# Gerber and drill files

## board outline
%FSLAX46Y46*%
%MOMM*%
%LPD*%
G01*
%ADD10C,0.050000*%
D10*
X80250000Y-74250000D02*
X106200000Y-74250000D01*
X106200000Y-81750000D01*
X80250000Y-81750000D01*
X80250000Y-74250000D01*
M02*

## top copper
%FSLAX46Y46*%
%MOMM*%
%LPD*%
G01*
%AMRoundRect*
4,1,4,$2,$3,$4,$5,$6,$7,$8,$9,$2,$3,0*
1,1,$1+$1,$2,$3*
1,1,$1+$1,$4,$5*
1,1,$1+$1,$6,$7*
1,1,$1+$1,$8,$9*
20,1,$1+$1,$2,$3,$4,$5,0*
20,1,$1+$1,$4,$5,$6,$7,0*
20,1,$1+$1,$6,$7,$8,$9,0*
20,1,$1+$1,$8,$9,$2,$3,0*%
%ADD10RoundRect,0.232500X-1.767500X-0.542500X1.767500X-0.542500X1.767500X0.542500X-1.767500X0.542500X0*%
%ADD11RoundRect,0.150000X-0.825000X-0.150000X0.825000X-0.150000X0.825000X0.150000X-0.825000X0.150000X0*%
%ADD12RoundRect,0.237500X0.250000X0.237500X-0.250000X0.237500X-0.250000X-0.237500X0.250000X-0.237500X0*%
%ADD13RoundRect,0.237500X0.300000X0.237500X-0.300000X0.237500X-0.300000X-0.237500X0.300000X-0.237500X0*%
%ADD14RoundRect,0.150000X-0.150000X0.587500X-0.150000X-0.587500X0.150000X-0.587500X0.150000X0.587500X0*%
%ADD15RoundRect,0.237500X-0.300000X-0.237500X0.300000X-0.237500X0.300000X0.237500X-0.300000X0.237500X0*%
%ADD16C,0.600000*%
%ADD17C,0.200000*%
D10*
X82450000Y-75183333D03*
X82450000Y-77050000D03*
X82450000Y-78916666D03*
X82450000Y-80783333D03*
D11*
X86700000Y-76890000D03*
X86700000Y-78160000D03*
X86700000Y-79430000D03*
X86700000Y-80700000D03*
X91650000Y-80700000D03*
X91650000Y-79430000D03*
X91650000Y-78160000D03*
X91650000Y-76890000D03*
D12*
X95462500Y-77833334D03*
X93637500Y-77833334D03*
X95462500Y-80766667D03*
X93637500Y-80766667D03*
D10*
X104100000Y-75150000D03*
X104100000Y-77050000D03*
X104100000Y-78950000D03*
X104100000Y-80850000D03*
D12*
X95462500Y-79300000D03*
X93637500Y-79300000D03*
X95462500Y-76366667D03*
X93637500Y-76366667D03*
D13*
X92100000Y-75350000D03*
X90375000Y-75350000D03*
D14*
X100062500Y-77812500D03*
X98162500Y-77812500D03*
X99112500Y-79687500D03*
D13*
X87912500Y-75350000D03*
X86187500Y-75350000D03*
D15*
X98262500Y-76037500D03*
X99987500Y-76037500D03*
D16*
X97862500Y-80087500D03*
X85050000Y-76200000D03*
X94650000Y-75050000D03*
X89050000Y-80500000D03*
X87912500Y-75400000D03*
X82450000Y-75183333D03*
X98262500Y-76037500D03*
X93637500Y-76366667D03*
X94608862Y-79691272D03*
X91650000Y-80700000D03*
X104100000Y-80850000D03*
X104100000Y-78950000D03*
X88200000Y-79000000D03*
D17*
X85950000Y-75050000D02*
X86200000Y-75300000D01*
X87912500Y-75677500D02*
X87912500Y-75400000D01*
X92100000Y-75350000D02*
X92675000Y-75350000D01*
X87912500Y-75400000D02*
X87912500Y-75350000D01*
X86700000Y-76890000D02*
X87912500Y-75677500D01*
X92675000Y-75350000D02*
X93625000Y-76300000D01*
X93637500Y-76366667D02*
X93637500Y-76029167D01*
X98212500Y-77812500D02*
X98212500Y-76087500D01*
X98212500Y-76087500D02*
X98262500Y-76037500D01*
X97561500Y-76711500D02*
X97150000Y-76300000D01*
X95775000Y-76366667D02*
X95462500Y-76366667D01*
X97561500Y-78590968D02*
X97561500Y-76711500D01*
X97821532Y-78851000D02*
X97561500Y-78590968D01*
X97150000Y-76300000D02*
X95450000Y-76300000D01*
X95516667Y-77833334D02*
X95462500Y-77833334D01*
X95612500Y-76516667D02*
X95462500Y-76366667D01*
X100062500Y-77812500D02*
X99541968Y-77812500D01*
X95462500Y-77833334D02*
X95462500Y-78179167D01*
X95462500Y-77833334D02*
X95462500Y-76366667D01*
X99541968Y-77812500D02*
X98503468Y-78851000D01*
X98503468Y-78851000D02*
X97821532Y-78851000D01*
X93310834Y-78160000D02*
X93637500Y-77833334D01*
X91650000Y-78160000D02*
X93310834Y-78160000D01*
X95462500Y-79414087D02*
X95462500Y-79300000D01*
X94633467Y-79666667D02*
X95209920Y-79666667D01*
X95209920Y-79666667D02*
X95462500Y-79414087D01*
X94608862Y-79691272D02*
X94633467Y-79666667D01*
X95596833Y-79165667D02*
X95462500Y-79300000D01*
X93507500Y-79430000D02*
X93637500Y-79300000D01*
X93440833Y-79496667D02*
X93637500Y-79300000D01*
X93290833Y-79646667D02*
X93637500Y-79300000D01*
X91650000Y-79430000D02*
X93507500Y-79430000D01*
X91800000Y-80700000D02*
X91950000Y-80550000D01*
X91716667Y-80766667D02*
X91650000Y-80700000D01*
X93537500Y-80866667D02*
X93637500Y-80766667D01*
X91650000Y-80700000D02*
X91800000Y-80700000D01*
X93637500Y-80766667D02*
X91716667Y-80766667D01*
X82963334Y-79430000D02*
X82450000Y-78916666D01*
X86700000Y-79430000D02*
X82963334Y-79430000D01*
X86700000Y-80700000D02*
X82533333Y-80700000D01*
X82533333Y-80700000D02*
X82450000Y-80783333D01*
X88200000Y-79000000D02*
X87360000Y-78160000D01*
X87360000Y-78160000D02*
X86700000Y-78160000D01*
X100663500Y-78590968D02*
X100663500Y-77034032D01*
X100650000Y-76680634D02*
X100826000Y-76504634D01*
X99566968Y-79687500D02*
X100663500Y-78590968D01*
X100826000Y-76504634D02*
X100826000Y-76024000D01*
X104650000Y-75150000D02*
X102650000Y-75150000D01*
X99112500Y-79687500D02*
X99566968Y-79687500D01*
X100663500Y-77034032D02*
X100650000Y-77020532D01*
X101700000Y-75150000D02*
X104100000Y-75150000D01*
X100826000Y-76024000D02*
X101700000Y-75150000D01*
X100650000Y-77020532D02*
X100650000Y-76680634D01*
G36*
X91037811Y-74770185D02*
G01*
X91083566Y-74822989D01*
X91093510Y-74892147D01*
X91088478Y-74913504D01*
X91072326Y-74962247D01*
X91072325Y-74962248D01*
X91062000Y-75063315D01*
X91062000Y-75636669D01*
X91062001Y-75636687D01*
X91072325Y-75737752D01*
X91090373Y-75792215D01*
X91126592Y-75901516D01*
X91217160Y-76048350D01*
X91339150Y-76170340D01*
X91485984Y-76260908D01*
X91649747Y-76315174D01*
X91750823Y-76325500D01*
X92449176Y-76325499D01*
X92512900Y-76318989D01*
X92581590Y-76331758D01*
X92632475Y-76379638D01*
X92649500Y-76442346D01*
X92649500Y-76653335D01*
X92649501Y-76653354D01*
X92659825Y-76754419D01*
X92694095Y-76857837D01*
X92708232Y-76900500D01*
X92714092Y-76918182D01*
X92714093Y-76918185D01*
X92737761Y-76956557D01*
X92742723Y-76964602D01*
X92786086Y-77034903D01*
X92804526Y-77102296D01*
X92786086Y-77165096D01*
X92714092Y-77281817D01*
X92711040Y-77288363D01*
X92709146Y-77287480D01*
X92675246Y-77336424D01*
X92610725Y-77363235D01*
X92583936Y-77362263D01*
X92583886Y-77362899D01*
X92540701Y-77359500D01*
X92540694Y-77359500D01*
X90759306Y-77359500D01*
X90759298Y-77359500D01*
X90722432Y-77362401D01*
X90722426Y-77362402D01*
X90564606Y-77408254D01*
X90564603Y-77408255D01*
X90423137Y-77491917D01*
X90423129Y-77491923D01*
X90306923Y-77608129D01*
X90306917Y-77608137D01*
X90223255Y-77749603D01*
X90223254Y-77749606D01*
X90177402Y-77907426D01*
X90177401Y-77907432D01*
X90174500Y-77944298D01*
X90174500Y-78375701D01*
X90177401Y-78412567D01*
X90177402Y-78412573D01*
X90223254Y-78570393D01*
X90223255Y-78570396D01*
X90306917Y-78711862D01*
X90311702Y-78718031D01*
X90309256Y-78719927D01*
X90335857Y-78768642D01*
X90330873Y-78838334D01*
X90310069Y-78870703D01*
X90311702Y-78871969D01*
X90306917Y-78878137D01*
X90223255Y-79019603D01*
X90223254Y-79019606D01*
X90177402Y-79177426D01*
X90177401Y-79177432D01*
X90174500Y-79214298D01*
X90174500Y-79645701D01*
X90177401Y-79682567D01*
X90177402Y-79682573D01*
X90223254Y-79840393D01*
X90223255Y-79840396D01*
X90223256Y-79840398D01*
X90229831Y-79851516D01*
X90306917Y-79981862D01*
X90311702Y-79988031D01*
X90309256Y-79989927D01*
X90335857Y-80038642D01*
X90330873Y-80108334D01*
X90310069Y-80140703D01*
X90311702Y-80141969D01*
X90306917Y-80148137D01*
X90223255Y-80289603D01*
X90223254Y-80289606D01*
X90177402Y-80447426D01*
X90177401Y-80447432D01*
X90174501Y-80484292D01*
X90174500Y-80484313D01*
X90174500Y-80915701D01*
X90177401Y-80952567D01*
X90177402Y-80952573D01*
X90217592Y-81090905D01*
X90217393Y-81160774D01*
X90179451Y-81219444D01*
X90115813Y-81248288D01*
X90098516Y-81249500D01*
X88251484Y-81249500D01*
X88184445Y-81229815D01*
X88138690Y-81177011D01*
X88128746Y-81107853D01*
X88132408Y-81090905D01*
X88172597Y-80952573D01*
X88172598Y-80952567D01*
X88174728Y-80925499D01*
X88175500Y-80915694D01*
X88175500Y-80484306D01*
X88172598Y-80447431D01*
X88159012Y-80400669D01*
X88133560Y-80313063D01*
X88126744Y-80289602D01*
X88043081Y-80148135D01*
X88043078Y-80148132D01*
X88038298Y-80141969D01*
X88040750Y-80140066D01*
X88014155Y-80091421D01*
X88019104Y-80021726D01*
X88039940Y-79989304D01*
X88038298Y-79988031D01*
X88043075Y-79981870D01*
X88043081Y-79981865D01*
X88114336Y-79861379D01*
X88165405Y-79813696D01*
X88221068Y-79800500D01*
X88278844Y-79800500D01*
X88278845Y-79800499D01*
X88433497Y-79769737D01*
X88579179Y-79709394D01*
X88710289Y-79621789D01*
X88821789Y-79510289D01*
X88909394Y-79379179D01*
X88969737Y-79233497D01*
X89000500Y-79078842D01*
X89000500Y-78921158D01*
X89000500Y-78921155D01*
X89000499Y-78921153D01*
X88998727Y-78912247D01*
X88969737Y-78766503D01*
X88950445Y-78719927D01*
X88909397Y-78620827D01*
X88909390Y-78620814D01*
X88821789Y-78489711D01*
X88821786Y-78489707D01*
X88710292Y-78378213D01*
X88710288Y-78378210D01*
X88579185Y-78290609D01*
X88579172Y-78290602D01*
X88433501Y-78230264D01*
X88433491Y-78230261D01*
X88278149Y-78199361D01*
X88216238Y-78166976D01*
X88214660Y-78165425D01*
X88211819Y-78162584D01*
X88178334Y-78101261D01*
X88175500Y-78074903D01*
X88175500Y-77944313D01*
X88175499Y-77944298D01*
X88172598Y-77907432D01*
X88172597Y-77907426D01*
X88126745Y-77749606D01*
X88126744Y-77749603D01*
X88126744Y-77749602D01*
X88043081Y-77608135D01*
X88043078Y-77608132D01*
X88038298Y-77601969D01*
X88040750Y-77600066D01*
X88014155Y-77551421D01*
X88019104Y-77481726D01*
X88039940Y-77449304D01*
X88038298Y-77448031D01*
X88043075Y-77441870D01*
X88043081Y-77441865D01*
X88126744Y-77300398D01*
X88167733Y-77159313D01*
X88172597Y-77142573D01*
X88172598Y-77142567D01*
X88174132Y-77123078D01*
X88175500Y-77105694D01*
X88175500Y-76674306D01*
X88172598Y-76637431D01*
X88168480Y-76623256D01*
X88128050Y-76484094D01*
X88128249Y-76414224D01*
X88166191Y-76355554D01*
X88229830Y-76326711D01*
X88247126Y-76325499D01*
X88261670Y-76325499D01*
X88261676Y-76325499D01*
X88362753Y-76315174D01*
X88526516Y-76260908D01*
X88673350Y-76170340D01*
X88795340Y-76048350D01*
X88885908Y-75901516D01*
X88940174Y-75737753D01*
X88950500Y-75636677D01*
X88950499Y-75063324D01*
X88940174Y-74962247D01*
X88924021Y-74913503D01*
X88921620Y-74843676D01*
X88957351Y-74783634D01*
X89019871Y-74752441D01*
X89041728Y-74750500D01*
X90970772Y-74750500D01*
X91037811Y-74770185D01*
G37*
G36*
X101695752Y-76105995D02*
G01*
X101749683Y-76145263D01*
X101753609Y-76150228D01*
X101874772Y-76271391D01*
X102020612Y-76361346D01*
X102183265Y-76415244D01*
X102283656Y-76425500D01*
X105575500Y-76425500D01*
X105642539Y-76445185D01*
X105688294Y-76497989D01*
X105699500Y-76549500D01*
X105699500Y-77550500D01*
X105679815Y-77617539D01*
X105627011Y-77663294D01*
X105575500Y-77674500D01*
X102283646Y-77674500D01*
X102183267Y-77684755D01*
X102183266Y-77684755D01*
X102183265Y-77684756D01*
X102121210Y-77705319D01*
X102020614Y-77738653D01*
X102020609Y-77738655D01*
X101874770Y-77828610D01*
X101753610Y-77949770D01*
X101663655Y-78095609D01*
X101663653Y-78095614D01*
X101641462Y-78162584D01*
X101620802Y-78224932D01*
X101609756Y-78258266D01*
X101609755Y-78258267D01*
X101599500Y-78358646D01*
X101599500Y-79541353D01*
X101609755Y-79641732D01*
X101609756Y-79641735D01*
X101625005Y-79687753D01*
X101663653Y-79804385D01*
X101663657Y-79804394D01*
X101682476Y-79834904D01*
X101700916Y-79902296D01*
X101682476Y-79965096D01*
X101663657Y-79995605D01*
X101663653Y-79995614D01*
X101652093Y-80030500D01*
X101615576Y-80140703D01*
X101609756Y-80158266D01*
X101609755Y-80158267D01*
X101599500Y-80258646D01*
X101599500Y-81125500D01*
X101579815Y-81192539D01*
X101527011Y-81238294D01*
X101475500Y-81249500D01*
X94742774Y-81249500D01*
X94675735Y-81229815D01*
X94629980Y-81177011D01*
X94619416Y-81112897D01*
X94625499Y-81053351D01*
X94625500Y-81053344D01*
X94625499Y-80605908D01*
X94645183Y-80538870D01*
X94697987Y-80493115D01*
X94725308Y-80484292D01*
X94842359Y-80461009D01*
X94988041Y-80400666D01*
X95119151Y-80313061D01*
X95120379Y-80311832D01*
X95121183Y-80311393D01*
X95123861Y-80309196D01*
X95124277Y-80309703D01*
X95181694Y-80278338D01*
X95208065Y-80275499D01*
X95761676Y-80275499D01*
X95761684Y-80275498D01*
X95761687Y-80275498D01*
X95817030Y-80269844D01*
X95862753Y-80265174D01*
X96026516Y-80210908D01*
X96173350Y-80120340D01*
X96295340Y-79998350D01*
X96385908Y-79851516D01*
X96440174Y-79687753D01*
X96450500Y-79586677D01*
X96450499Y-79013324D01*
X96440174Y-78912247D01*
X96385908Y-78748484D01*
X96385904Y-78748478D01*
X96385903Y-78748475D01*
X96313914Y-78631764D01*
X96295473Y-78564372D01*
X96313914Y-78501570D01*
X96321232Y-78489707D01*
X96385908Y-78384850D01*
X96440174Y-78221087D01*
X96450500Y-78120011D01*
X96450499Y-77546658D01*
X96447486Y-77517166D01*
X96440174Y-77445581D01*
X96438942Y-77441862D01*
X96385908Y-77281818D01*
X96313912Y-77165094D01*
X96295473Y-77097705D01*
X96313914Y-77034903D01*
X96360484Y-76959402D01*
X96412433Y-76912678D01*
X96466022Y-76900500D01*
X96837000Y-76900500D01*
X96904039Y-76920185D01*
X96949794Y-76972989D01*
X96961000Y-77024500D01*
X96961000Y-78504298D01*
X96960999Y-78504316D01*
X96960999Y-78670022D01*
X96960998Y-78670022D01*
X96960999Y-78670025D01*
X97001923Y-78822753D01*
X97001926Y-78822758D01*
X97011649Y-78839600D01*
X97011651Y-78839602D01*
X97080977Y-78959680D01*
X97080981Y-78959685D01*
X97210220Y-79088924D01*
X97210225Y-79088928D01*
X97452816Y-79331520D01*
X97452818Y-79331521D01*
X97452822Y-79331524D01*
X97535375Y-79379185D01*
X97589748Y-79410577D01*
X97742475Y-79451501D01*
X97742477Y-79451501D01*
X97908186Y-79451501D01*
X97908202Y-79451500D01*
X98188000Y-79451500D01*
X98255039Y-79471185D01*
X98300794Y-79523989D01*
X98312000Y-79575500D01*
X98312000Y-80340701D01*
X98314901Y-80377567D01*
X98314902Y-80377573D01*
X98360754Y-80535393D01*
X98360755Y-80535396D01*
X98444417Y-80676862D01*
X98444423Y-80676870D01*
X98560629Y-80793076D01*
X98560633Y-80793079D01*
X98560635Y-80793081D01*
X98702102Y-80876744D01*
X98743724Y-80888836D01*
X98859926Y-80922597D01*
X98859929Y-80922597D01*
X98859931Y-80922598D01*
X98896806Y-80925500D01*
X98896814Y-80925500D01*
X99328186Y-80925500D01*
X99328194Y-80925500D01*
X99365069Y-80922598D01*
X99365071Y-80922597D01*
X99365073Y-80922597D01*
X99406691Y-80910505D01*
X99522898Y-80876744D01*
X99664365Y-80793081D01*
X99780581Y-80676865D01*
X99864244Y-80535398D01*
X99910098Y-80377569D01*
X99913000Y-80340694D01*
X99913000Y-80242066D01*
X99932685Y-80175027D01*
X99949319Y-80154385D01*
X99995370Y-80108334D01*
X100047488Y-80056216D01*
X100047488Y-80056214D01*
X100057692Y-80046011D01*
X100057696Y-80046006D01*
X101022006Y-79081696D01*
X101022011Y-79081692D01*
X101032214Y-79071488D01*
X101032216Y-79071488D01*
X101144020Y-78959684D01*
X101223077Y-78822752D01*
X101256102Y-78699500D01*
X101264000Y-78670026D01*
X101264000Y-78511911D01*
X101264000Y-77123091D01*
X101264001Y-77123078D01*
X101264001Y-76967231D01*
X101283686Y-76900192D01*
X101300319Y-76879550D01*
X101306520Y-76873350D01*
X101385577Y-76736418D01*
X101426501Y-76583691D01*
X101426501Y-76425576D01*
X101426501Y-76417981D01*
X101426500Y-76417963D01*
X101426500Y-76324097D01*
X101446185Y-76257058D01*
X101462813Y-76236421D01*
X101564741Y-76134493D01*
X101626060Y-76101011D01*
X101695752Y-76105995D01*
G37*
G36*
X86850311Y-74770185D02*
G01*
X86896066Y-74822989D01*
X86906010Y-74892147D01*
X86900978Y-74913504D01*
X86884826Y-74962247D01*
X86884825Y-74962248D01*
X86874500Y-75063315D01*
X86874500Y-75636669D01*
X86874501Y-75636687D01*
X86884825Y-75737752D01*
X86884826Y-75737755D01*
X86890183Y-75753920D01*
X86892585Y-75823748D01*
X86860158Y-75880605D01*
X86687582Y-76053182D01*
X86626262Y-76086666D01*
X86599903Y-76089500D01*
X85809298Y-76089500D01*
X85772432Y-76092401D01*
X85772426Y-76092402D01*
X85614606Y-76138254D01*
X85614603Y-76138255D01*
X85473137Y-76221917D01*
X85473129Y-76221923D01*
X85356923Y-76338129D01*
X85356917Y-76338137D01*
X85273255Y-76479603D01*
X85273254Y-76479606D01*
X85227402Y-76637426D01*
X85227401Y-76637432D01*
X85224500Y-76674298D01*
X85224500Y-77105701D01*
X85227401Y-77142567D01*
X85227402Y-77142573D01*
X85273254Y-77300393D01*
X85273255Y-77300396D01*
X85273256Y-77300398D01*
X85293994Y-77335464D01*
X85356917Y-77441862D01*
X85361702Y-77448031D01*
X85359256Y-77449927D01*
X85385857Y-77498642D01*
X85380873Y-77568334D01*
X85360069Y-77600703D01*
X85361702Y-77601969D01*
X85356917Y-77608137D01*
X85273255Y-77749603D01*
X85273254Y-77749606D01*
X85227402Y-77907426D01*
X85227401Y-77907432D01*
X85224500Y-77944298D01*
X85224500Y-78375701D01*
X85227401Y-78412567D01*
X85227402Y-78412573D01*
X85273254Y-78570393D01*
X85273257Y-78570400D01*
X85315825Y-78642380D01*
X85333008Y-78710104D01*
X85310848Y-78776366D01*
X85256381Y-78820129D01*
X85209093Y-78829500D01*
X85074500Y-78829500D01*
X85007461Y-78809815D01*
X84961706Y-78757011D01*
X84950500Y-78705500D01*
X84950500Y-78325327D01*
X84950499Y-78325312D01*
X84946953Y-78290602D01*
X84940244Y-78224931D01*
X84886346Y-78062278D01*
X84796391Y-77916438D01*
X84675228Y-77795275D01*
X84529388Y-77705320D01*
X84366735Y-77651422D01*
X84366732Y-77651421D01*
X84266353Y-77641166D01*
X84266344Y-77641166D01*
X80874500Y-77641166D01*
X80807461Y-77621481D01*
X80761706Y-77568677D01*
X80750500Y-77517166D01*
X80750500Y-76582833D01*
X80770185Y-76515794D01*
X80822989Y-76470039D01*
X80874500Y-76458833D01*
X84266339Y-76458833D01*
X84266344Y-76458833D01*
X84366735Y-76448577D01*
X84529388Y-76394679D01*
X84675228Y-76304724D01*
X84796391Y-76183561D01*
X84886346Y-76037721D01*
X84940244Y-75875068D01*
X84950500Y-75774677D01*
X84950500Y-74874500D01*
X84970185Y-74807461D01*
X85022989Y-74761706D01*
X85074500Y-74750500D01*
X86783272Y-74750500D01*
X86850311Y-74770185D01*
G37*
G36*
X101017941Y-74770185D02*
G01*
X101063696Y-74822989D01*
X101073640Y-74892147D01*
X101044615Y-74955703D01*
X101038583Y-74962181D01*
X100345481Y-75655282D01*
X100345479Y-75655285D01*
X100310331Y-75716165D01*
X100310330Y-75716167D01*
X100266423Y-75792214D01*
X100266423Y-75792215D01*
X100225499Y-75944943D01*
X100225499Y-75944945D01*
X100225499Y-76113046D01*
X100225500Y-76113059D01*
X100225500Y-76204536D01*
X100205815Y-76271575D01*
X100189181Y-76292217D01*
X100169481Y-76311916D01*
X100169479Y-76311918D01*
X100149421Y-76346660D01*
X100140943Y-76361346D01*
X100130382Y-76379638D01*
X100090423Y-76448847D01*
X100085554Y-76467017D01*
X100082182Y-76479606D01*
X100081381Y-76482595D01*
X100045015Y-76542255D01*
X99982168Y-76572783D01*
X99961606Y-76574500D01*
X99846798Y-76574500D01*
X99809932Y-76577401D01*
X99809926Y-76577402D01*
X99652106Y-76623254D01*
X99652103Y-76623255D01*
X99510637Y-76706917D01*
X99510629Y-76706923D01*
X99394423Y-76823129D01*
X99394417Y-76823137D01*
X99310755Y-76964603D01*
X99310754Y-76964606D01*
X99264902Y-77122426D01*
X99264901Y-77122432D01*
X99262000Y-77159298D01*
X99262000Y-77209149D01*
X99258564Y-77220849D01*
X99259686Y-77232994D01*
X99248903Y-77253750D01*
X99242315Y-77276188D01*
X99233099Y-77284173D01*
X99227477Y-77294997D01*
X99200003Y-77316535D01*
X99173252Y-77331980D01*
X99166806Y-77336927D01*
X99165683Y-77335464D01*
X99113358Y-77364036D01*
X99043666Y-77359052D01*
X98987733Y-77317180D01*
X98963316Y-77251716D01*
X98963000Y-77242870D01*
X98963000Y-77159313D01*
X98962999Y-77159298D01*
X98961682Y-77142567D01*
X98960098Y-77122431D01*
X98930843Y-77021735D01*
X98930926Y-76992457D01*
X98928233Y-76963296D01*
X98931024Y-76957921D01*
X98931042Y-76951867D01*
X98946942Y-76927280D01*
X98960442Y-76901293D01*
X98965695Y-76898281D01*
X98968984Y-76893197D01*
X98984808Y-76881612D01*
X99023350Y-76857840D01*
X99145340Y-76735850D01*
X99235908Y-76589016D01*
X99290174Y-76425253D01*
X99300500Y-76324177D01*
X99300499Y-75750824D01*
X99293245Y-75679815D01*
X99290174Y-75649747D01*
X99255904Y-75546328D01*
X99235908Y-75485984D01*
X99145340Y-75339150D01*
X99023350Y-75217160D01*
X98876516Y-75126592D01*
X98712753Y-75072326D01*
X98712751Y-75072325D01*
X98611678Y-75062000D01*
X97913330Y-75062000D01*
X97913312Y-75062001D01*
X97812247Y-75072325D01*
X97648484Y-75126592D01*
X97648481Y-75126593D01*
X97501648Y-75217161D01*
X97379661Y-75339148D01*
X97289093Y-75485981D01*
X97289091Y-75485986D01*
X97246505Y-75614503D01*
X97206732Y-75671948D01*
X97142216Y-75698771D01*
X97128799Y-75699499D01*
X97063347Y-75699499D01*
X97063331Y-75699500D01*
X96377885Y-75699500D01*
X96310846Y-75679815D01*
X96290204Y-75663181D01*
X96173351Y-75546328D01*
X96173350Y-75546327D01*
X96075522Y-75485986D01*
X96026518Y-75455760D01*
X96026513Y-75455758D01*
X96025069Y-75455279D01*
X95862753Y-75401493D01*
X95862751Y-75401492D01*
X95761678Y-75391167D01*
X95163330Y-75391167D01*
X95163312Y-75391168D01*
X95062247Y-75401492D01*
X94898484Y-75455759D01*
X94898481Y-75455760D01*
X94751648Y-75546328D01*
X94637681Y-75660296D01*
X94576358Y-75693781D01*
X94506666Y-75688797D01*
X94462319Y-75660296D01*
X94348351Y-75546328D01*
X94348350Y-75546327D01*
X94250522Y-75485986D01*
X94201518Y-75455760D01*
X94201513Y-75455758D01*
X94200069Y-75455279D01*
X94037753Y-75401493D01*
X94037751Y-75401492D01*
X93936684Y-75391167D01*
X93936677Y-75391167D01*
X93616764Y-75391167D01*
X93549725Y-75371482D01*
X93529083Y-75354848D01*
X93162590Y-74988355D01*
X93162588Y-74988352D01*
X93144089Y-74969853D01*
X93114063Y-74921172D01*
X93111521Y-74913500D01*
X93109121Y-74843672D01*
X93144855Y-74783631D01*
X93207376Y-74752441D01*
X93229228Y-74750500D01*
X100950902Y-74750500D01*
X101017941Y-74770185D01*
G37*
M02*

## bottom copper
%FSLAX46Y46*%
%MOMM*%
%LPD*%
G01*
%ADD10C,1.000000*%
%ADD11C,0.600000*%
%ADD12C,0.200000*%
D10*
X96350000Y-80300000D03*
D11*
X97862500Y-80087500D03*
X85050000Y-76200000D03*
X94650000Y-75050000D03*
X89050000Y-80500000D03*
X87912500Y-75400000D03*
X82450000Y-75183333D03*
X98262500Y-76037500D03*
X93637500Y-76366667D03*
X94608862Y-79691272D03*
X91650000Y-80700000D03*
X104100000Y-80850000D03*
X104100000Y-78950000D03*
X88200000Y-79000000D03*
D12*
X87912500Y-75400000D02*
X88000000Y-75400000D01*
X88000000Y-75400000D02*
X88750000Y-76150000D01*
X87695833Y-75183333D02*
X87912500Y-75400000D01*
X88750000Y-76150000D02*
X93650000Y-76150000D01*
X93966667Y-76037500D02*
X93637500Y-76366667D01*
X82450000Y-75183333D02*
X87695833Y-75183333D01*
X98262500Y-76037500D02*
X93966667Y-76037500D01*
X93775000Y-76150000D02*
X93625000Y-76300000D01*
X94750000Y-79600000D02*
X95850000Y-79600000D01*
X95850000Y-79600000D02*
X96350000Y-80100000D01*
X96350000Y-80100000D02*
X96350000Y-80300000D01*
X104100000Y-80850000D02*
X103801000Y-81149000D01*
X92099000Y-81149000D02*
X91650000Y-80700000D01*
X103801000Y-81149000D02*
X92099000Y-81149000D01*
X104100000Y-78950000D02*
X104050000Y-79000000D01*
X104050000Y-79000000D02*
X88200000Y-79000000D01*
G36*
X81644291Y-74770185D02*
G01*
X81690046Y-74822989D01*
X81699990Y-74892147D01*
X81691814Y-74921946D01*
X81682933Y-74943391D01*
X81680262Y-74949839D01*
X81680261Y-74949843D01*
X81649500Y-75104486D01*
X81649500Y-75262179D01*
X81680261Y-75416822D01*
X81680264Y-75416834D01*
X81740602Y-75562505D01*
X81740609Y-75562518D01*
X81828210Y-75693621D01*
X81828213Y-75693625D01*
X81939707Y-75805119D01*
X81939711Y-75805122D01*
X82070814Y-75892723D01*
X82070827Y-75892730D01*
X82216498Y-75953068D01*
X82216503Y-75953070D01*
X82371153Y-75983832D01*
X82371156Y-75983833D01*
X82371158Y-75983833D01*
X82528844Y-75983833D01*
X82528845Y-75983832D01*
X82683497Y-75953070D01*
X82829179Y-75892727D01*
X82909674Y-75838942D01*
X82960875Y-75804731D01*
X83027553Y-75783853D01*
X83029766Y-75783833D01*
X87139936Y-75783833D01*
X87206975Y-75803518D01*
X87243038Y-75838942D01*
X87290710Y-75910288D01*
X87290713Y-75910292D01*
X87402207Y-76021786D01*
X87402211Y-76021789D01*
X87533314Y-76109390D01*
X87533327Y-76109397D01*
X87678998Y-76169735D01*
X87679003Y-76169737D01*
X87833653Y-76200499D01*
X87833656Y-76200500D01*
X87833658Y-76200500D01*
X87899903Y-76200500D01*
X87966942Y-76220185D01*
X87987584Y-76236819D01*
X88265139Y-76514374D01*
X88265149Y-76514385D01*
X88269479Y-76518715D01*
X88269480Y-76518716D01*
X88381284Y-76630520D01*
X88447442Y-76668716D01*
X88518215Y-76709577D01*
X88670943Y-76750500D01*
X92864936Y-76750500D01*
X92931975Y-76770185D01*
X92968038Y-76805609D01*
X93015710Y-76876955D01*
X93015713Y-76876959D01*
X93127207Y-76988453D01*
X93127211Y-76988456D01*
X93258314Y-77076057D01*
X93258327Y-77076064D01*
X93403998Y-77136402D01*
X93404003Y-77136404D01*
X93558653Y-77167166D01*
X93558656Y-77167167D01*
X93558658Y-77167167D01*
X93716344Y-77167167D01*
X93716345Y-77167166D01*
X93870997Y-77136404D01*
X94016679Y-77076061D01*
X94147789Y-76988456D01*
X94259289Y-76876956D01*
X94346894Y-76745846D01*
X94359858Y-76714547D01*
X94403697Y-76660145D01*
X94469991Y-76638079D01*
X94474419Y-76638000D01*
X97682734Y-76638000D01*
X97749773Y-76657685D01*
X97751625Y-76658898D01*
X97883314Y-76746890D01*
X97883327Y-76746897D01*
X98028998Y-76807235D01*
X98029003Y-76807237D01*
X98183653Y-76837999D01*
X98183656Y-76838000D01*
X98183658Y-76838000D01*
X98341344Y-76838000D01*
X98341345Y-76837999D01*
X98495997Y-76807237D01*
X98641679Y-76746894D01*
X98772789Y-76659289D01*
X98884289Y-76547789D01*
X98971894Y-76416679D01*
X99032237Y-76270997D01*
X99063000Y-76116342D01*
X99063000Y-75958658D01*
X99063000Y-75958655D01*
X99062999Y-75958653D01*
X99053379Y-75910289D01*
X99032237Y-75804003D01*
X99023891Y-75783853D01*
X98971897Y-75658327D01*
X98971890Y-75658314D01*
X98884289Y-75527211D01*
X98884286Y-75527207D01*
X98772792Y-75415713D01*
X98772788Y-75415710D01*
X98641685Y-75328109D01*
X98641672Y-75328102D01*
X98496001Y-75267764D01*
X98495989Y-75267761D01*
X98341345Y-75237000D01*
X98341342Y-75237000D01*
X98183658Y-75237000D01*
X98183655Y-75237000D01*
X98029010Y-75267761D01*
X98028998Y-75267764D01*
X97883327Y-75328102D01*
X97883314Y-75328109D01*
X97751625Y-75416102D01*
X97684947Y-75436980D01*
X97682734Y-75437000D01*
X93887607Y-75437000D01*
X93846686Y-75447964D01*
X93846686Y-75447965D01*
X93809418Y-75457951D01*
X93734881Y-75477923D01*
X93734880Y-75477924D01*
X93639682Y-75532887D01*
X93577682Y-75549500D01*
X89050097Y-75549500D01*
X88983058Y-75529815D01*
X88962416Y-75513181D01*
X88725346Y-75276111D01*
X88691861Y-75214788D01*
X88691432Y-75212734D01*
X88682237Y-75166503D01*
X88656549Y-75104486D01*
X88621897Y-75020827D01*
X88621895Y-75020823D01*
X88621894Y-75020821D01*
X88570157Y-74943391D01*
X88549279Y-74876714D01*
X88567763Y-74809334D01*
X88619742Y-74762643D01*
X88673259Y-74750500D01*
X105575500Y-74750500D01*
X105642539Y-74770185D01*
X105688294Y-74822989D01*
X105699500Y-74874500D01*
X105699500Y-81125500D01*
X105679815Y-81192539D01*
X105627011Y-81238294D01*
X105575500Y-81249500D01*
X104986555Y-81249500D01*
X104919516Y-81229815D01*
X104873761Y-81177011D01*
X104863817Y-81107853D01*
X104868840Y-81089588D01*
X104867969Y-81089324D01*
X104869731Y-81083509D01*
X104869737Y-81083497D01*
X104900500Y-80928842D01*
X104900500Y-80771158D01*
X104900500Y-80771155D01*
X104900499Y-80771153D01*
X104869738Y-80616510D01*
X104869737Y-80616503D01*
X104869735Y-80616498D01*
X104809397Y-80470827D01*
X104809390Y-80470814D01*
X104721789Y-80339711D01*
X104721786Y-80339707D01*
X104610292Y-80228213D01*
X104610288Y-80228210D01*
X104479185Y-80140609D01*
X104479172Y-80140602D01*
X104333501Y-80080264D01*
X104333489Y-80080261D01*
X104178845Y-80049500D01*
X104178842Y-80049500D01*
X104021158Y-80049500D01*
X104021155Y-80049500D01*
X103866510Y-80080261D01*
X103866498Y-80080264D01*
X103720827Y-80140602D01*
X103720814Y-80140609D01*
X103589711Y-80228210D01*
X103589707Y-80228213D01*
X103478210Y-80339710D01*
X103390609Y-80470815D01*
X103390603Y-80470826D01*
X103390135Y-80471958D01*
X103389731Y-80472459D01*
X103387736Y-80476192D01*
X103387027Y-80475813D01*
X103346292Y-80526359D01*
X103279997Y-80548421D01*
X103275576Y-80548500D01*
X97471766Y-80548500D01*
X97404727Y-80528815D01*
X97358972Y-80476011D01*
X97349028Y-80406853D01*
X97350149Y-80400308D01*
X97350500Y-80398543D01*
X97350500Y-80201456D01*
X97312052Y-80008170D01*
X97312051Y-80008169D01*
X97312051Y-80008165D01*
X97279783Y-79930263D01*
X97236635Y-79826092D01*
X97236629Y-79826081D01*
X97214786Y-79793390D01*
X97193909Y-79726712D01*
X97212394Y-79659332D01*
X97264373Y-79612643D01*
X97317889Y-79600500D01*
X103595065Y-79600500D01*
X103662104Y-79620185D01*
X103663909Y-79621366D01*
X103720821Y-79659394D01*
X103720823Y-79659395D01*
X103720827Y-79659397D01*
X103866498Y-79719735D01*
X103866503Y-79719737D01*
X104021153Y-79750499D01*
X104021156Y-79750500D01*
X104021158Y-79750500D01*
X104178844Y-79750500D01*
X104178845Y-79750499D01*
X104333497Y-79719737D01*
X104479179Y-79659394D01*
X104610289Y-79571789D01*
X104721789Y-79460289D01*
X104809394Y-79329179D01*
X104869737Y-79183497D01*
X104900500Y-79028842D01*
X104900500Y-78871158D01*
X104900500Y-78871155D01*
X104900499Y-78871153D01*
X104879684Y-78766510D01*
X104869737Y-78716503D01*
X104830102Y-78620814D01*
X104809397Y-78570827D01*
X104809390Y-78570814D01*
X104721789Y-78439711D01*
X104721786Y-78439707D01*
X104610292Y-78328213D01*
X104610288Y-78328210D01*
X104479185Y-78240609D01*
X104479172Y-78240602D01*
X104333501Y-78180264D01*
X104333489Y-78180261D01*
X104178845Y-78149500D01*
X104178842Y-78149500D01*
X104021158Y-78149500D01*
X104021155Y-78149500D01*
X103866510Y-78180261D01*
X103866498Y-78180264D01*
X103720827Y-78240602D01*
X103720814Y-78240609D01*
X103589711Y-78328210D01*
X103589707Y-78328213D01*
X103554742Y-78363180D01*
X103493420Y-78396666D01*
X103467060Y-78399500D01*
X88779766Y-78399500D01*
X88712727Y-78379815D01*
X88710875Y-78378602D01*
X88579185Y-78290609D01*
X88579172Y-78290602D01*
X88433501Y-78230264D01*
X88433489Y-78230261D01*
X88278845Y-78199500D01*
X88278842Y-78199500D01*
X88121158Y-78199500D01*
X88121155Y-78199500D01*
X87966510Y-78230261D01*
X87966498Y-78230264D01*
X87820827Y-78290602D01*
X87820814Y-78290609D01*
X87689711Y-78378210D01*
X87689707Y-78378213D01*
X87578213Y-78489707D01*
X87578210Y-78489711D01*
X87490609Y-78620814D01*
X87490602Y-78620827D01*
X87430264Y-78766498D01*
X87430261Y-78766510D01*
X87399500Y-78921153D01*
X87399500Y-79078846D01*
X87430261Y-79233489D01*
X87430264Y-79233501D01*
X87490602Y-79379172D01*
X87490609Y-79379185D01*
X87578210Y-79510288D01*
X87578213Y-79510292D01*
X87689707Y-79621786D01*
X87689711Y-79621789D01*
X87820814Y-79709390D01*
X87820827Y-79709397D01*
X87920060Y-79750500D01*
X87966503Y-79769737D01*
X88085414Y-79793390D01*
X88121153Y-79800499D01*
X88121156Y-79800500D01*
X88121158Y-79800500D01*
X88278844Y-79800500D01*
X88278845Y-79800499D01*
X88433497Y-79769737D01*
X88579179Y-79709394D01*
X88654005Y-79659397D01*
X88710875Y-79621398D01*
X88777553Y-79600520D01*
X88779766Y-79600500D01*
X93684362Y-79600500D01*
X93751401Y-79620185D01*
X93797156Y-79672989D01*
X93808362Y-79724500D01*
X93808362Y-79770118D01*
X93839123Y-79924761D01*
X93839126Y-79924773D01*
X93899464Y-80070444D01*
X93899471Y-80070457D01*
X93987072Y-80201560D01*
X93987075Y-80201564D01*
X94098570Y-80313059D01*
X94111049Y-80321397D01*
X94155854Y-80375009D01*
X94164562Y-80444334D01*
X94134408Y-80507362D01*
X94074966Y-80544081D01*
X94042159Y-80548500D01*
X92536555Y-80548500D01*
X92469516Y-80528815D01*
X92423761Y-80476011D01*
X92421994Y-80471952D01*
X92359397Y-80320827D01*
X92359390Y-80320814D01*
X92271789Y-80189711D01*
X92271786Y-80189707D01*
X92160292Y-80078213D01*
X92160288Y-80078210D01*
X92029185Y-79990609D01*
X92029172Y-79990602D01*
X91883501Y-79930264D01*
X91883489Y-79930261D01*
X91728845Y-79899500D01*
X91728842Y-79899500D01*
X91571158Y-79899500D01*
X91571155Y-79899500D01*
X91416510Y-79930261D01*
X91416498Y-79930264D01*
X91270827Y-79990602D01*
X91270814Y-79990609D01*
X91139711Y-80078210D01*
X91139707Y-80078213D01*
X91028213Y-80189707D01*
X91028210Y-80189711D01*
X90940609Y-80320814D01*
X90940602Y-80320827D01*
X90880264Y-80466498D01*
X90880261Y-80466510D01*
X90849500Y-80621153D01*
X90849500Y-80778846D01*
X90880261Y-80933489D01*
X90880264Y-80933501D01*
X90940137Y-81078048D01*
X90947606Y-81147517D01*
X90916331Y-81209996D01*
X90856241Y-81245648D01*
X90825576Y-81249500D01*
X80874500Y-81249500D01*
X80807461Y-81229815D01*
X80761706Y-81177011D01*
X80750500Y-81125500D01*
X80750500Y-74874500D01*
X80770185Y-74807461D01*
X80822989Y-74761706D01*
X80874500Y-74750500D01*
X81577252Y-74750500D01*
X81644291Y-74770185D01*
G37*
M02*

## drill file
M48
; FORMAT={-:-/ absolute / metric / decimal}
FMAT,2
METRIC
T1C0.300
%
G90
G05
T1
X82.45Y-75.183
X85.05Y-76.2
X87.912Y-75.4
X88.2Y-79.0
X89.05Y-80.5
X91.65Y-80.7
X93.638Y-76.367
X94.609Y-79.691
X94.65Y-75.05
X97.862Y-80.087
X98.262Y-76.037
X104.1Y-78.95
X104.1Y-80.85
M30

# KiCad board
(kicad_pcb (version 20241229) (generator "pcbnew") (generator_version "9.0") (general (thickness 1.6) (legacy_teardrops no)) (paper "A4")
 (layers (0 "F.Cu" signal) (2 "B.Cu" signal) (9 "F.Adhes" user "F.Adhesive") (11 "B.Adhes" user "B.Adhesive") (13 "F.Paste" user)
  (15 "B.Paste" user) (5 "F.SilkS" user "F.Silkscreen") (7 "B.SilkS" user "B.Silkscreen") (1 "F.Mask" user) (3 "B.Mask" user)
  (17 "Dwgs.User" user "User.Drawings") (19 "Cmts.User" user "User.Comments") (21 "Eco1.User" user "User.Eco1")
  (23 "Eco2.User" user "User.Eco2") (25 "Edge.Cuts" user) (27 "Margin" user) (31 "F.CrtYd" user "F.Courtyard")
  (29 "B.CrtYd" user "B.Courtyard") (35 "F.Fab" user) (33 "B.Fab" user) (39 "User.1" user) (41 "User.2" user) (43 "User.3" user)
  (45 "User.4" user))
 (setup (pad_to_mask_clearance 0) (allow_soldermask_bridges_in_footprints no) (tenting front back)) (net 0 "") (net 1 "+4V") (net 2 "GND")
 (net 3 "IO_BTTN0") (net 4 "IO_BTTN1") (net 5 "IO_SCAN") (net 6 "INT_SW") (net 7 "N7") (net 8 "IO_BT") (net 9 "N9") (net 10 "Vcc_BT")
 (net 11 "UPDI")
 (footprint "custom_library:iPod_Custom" (layer "F.Cu") (at 83 82.433333)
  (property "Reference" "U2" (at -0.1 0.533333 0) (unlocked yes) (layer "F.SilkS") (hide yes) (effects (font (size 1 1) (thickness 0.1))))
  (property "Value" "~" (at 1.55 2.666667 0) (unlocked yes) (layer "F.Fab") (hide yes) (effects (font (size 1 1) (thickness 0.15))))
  (pad "1" connect roundrect (at -0.55 -7.25) (size 4 1.55) (layers "F.Cu" "F.Mask") (roundrect_rratio 0.15) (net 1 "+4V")
   (thermal_bridge_angle 45))
  (pad "2" connect roundrect (at -0.55 -5.383333) (size 4 1.55) (layers "F.Cu" "F.Mask") (roundrect_rratio 0.15) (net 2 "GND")
   (thermal_bridge_angle 45))
  (pad "3" connect roundrect (at -0.55 -3.516667) (size 4 1.55) (layers "F.Cu" "F.Mask") (roundrect_rratio 0.15) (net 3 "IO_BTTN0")
   (thermal_bridge_angle 45))
  (pad "4" connect roundrect (at -0.55 -1.65) (size 4 1.55) (layers "F.Cu" "F.Mask") (roundrect_rratio 0.15) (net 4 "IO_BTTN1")
   (thermal_bridge_angle 45)))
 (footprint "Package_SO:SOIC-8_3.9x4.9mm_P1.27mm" (layer "F.Cu") (at 89.175 78.795)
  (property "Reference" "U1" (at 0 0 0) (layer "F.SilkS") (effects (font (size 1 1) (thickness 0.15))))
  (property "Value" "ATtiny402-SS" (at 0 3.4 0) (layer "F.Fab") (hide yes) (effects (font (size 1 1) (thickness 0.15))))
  (pad "1" smd roundrect (at -2.475 -1.905) (size 1.95 0.6) (layers "F.Cu" "F.Mask" "F.Paste") (roundrect_rratio 0.25) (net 1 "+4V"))
  (pad "2" smd roundrect (at -2.475 -0.635) (size 1.95 0.6) (layers "F.Cu" "F.Mask" "F.Paste") (roundrect_rratio 0.25) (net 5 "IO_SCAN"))
  (pad "3" smd roundrect (at -2.475 0.635) (size 1.95 0.6) (layers "F.Cu" "F.Mask" "F.Paste") (roundrect_rratio 0.25) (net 3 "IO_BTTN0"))
  (pad "4" smd roundrect (at -2.475 1.905) (size 1.95 0.6) (layers "F.Cu" "F.Mask" "F.Paste") (roundrect_rratio 0.25) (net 4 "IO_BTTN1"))
  (pad "5" smd roundrect (at 2.475 1.905) (size 1.95 0.6) (layers "F.Cu" "F.Mask" "F.Paste") (roundrect_rratio 0.25) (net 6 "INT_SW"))
  (pad "6" smd roundrect (at 2.475 0.635) (size 1.95 0.6) (layers "F.Cu" "F.Mask" "F.Paste") (roundrect_rratio 0.25) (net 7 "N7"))
  (pad "7" smd roundrect (at 2.475 -0.635) (size 1.95 0.6) (layers "F.Cu" "F.Mask" "F.Paste") (roundrect_rratio 0.25) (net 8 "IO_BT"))
  (pad "8" smd roundrect (at 2.475 -1.905) (size 1.95 0.6) (layers "F.Cu" "F.Mask" "F.Paste") (roundrect_rratio 0.25) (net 2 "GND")))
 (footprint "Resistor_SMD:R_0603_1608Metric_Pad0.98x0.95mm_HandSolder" (layer "F.Cu") (at 94.55 77.833334 180)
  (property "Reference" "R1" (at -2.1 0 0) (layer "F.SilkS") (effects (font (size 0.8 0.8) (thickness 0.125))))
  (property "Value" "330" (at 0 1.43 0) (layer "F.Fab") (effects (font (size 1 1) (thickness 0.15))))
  (pad "1" smd roundrect (at -0.9125 0 180) (size 0.975 0.95) (layers "F.Cu" "F.Mask" "F.Paste") (roundrect_rratio 0.25) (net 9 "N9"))
  (pad "2" smd roundrect (at 0.9125 0 180) (size 0.975 0.95) (layers "F.Cu" "F.Mask" "F.Paste") (roundrect_rratio 0.25) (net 8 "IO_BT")))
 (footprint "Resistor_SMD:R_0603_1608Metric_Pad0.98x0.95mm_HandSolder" (layer "F.Cu") (at 94.55 80.766667 180)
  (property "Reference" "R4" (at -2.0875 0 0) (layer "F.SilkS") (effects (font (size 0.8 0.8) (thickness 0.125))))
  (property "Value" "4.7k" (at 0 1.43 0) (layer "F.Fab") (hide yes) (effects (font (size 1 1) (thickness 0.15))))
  (pad "1" smd roundrect (at -0.9125 0 180) (size 0.975 0.95) (layers "F.Cu" "F.Mask" "F.Paste") (roundrect_rratio 0.25) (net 2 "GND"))
  (pad "2" smd roundrect (at 0.9125 0 180) (size 0.975 0.95) (layers "F.Cu" "F.Mask" "F.Paste") (roundrect_rratio 0.25) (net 6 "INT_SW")))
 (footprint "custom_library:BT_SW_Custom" (layer "F.Cu") (at 103.4 82.35)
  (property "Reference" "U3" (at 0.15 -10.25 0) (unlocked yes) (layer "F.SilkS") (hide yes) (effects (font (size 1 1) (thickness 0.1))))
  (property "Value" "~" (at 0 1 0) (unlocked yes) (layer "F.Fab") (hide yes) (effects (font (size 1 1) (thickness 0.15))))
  (pad "1" connect roundrect (at 0.7 -7.2) (size 4 1.55) (layers "F.Cu" "F.Mask") (roundrect_rratio 0.15) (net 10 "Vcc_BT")
   (thermal_bridge_angle 45))
  (pad "2" connect roundrect (at 0.7 -5.3) (size 4 1.55) (layers "F.Cu" "F.Mask") (roundrect_rratio 0.15) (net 2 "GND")
   (thermal_bridge_angle 45))
  (pad "3" connect roundrect (at 0.7 -3.4) (size 4 1.55) (layers "F.Cu" "F.Mask") (roundrect_rratio 0.15) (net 5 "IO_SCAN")
   (thermal_bridge_angle 45))
  (pad "4" connect roundrect (at 0.7 -1.5) (size 4 1.55) (layers "F.Cu" "F.Mask") (roundrect_rratio 0.15) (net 6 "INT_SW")
   (thermal_bridge_angle 45)))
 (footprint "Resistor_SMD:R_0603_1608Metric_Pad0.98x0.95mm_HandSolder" (layer "F.Cu") (at 94.55 79.3 180)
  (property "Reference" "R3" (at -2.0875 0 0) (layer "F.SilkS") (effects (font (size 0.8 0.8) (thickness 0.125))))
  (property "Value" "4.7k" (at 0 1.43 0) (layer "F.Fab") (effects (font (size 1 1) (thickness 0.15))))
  (pad "1" smd roundrect (at -0.9125 0 180) (size 0.975 0.95) (layers "F.Cu" "F.Mask" "F.Paste") (roundrect_rratio 0.25) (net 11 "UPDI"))
  (pad "2" smd roundrect (at 0.9125 0 180) (size 0.975 0.95) (layers "F.Cu" "F.Mask" "F.Paste") (roundrect_rratio 0.25) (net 7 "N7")))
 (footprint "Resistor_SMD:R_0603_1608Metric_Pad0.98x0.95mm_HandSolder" (layer "F.Cu") (at 94.55 76.366667 180)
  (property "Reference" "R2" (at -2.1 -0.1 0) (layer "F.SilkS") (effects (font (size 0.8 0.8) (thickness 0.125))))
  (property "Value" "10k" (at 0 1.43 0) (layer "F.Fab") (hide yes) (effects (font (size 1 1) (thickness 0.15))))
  (pad "1" smd roundrect (at -0.9125 0 180) (size 0.975 0.95) (layers "F.Cu" "F.Mask" "F.Paste") (roundrect_rratio 0.25) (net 9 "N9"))
  (pad "2" smd roundrect (at 0.9125 0 180) (size 0.975 0.95) (layers "F.Cu" "F.Mask" "F.Paste") (roundrect_rratio 0.25) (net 1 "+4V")))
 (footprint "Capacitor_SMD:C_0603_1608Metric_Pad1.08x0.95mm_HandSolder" (layer "F.Cu") (at 91.2375 75.35 180)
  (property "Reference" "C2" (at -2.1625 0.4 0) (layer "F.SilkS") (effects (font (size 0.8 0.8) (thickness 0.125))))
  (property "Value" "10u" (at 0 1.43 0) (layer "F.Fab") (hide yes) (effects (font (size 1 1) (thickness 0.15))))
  (pad "1" smd roundrect (at -0.8625 0 180) (size 1.075 0.95) (layers "F.Cu" "F.Mask" "F.Paste") (roundrect_rratio 0.25) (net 1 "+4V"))
  (pad "2" smd roundrect (at 0.8625 0 180) (size 1.075 0.95) (layers "F.Cu" "F.Mask" "F.Paste") (roundrect_rratio 0.25) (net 2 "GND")))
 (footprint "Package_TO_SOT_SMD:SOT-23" (layer "F.Cu") (at 99.1125 78.75 -90)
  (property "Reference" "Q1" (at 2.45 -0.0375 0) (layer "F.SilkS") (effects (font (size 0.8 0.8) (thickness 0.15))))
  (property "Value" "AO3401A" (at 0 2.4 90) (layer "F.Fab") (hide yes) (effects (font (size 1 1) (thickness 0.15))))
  (pad "1" smd roundrect (at -0.9375 -0.95 270) (size 1.475 0.6) (layers "F.Cu" "F.Mask" "F.Paste") (roundrect_rratio 0.25) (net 9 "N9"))
  (pad "2" smd roundrect (at -0.9375 0.95 270) (size 1.475 0.6) (layers "F.Cu" "F.Mask" "F.Paste") (roundrect_rratio 0.25) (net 1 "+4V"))
  (pad "3" smd roundrect (at 0.9375 0 270) (size 1.475 0.6) (layers "F.Cu" "F.Mask" "F.Paste") (roundrect_rratio 0.25) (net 10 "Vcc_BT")))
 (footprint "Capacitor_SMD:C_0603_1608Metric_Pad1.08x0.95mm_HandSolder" (layer "F.Cu") (at 87.05 75.35 180)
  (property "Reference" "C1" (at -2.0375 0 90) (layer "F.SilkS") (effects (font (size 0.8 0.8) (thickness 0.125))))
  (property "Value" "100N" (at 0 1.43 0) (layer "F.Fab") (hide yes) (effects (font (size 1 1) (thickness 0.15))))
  (pad "1" smd roundrect (at -0.8625 0 180) (size 1.075 0.95) (layers "F.Cu" "F.Mask" "F.Paste") (roundrect_rratio 0.25) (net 1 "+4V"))
  (pad "2" smd roundrect (at 0.8625 0 180) (size 1.075 0.95) (layers "F.Cu" "F.Mask" "F.Paste") (roundrect_rratio 0.25) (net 2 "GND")))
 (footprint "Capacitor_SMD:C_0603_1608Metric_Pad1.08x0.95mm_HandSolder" (layer "F.Cu") (at 99.125 76.0375)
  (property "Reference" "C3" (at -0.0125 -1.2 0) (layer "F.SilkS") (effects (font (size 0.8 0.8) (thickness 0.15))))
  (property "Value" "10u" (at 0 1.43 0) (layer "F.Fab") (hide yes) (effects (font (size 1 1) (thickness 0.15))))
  (pad "1" smd roundrect (at -0.8625 0) (size 1.075 0.95) (layers "F.Cu" "F.Mask" "F.Paste") (roundrect_rratio 0.25) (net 1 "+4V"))
  (pad "2" smd roundrect (at 0.8625 0) (size 1.075 0.95) (layers "F.Cu" "F.Mask" "F.Paste") (roundrect_rratio 0.25) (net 2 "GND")))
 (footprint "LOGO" (layer "B.Cu") (at 84.3 77.8 180)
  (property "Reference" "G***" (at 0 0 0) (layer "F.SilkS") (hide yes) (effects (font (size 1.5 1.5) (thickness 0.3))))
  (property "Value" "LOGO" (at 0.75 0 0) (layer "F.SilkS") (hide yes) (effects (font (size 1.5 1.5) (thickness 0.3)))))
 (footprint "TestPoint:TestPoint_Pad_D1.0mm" (layer "B.Cu") (at 96.35 80.3 180)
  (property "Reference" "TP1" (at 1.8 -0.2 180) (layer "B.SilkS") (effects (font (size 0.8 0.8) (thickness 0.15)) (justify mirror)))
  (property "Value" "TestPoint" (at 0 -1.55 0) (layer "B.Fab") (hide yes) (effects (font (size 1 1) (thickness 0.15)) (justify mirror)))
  (pad "1" smd circle (at 0 0 180) (size 1 1) (layers "B.Cu" "B.Mask") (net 11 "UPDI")))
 (gr_rect (start 80.25 74.25) (end 106.2 81.75) (stroke (width 0.05) (type solid)) (fill no) (layer "Edge.Cuts"))
 (segment (start 85.95 75.05) (end 86.2 75.3) (width 0.2) (layer "F.Cu") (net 2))
 (via (at 97.8625 80.0875) (size 0.6) (drill 0.3) (layers "F.Cu" "B.Cu") (free yes) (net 2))
 (via (at 85.05 76.2) (size 0.6) (drill 0.3) (layers "F.Cu" "B.Cu") (free yes) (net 2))
 (via (at 94.65 75.05) (size 0.6) (drill 0.3) (layers "F.Cu" "B.Cu") (free yes) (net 2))
 (via (at 89.05 80.5) (size 0.6) (drill 0.3) (layers "F.Cu" "B.Cu") (free yes) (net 2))
 (segment (start 87.9125 75.6775) (end 87.9125 75.4) (width 0.2) (layer "F.Cu") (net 1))
 (segment (start 92.1 75.35) (end 92.675 75.35) (width 0.2) (layer "F.Cu") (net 1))
 (segment (start 87.9125 75.4) (end 87.9125 75.35) (width 0.2) (layer "F.Cu") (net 1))
 (segment (start 86.7 76.89) (end 87.9125 75.6775) (width 0.2) (layer "F.Cu") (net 1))
 (segment (start 92.675 75.35) (end 93.625 76.3) (width 0.2) (layer "F.Cu") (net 1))
 (segment (start 93.6375 76.366667) (end 93.6375 76.029167) (width 0.2) (layer "F.Cu") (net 1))
 (segment (start 98.2125 77.8125) (end 98.2125 76.0875) (width 0.2) (layer "F.Cu") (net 1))
 (segment (start 98.2125 76.0875) (end 98.2625 76.0375) (width 0.2) (layer "F.Cu") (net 1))
 (via (at 87.9125 75.4) (size 0.6) (drill 0.3) (layers "F.Cu" "B.Cu") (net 1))
 (via (at 82.45 75.183333) (size 0.6) (drill 0.3) (layers "F.Cu" "B.Cu") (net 1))
 (via (at 98.2625 76.0375) (size 0.6) (drill 0.3) (layers "F.Cu" "B.Cu") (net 1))
 (via (at 93.6375 76.366667) (size 0.6) (drill 0.3) (layers "F.Cu" "B.Cu") (free yes) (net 1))
 (segment (start 87.9125 75.4) (end 88 75.4) (width 0.2) (layer "B.Cu") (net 1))
 (segment (start 88 75.4) (end 88.75 76.15) (width 0.2) (layer "B.Cu") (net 1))
 (segment (start 87.695833 75.183333) (end 87.9125 75.4) (width 0.2) (layer "B.Cu") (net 1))
 (segment (start 88.75 76.15) (end 93.65 76.15) (width 0.2) (layer "B.Cu") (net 1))
 (segment (start 93.966667 76.0375) (end 93.6375 76.366667) (width 0.2) (layer "B.Cu") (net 1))
 (segment (start 82.45 75.183333) (end 87.695833 75.183333) (width 0.2) (layer "B.Cu") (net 1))
 (segment (start 98.2625 76.0375) (end 93.966667 76.0375) (width 0.2) (layer "B.Cu") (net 1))
 (segment (start 93.775 76.15) (end 93.625 76.3) (width 0.2) (layer "B.Cu") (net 1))
 (segment (start 97.5615 76.7115) (end 97.15 76.3) (width 0.2) (layer "F.Cu") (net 9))
 (segment (start 95.775 76.366667) (end 95.4625 76.366667) (width 0.2) (layer "F.Cu") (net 9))
 (segment (start 97.5615 78.590968) (end 97.5615 76.7115) (width 0.2) (layer "F.Cu") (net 9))
 (segment (start 97.821532 78.851) (end 97.5615 78.590968) (width 0.2) (layer "F.Cu") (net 9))
 (segment (start 97.15 76.3) (end 95.45 76.3) (width 0.2) (layer "F.Cu") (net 9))
 (segment (start 95.516667 77.833334) (end 95.4625 77.833334) (width 0.2) (layer "F.Cu") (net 9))
 (segment (start 95.6125 76.516667) (end 95.4625 76.366667) (width 0.2) (layer "F.Cu") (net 9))
 (segment (start 100.0625 77.8125) (end 99.541968 77.8125) (width 0.2) (layer "F.Cu") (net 9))
 (segment (start 95.4625 77.833334) (end 95.4625 78.179167) (width 0.2) (layer "F.Cu") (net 9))
 (segment (start 95.4625 77.833334) (end 95.4625 76.366667) (width 0.2) (layer "F.Cu") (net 9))
 (segment (start 99.541968 77.8125) (end 98.503468 78.851) (width 0.2) (layer "F.Cu") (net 9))
 (segment (start 98.503468 78.851) (end 97.821532 78.851) (width 0.2) (layer "F.Cu") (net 9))
 (segment (start 93.310834 78.16) (end 93.6375 77.833334) (width 0.2) (layer "F.Cu") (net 8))
 (segment (start 91.65 78.16) (end 93.310834 78.16) (width 0.2) (layer "F.Cu") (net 8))
 (segment (start 95.4625 79.414087) (end 95.4625 79.3) (width 0.2) (layer "F.Cu") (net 11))
 (segment (start 94.633467 79.666667) (end 95.20992 79.666667) (width 0.2) (layer "F.Cu") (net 11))
 (segment (start 95.20992 79.666667) (end 95.4625 79.414087) (width 0.2) (layer "F.Cu") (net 11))
 (segment (start 94.608862 79.691272) (end 94.633467 79.666667) (width 0.2) (layer "F.Cu") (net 11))
 (segment (start 95.596833 79.165667) (end 95.4625 79.3) (width 0.2) (layer "F.Cu") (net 11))
 (via (at 94.608862 79.691272) (size 0.6) (drill 0.3) (layers "F.Cu" "B.Cu") (free yes) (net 11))
 (segment (start 94.75 79.6) (end 95.85 79.6) (width 0.2) (layer "B.Cu") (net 11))
 (segment (start 95.85 79.6) (end 96.35 80.1) (width 0.2) (layer "B.Cu") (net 11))
 (segment (start 96.35 80.1) (end 96.35 80.3) (width 0.2) (layer "B.Cu") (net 11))
 (segment (start 93.5075 79.43) (end 93.6375 79.3) (width 0.2) (layer "F.Cu") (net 7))
 (segment (start 93.440833 79.496667) (end 93.6375 79.3) (width 0.2) (layer "F.Cu") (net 7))
 (segment (start 93.290833 79.646667) (end 93.6375 79.3) (width 0.2) (layer "F.Cu") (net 7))
 (segment (start 91.65 79.43) (end 93.5075 79.43) (width 0.2) (layer "F.Cu") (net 7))
 (segment (start 91.8 80.7) (end 91.95 80.55) (width 0.2) (layer "F.Cu") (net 6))
 (segment (start 91.716667 80.766667) (end 91.65 80.7) (width 0.2) (layer "F.Cu") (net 6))
 (segment (start 93.5375 80.866667) (end 93.6375 80.766667) (width 0.2) (layer "F.Cu") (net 6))
 (segment (start 91.65 80.7) (end 91.8 80.7) (width 0.2) (layer "F.Cu") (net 6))
 (segment (start 93.6375 80.766667) (end 91.716667 80.766667) (width 0.2) (layer "F.Cu") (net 6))
 (via (at 91.65 80.7) (size 0.6) (drill 0.3) (layers "F.Cu" "B.Cu") (free yes) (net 6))
 (via (at 104.1 80.85) (size 0.6) (drill 0.3) (layers "F.Cu" "B.Cu") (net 6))
 (segment (start 104.1 80.85) (end 103.801 81.149) (width 0.2) (layer "B.Cu") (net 6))
 (segment (start 92.099 81.149) (end 91.65 80.7) (width 0.2) (layer "B.Cu") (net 6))
 (segment (start 103.801 81.149) (end 92.099 81.149) (width 0.2) (layer "B.Cu") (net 6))
 (segment (start 82.963334 79.43) (end 82.45 78.916666) (width 0.2) (layer "F.Cu") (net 3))
 (segment (start 86.7 79.43) (end 82.963334 79.43) (width 0.2) (layer "F.Cu") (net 3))
 (segment (start 86.7 80.7) (end 82.533333 80.7) (width 0.2) (layer "F.Cu") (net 4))
 (segment (start 82.533333 80.7) (end 82.45 80.783333) (width 0.2) (layer "F.Cu") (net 4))
 (segment (start 88.2 79) (end 87.36 78.16) (width 0.2) (layer "F.Cu") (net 5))
 (segment (start 87.36 78.16) (end 86.7 78.16) (width 0.2) (layer "F.Cu") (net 5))
 (via (at 104.1 78.95) (size 0.6) (drill 0.3) (layers "F.Cu" "B.Cu") (free yes) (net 5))
 (via (at 88.2 79) (size 0.6) (drill 0.3) (layers "F.Cu" "B.Cu") (free yes) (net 5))
 (segment (start 104.1 78.95) (end 104.05 79) (width 0.2) (layer "B.Cu") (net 5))
 (segment (start 104.05 79) (end 88.2 79) (width 0.2) (layer "B.Cu") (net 5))
 (segment (start 100.6635 78.590968) (end 100.6635 77.034032) (width 0.2) (layer "F.Cu") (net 10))
 (segment (start 100.65 76.680634) (end 100.826 76.504634) (width 0.2) (layer "F.Cu") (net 10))
 (segment (start 99.566968 79.6875) (end 100.6635 78.590968) (width 0.2) (layer "F.Cu") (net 10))
 (segment (start 100.826 76.504634) (end 100.826 76.024) (width 0.2) (layer "F.Cu") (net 10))
 (segment (start 104.65 75.15) (end 102.65 75.15) (width 0.2) (layer "F.Cu") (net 10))
 (segment (start 99.1125 79.6875) (end 99.566968 79.6875) (width 0.2) (layer "F.Cu") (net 10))
 (segment (start 100.6635 77.034032) (end 100.65 77.020532) (width 0.2) (layer "F.Cu") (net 10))
 (segment (start 101.7 75.15) (end 104.1 75.15) (width 0.2) (layer "F.Cu") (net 10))
 (segment (start 100.826 76.024) (end 101.7 75.15) (width 0.2) (layer "F.Cu") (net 10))
 (segment (start 100.65 77.020532) (end 100.65 76.680634) (width 0.2) (layer "F.Cu") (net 10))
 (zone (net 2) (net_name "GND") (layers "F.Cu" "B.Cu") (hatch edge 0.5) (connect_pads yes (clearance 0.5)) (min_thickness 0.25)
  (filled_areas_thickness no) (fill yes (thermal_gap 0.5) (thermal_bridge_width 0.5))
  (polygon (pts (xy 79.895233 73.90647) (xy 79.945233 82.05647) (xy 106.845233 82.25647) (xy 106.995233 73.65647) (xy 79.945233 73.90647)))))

